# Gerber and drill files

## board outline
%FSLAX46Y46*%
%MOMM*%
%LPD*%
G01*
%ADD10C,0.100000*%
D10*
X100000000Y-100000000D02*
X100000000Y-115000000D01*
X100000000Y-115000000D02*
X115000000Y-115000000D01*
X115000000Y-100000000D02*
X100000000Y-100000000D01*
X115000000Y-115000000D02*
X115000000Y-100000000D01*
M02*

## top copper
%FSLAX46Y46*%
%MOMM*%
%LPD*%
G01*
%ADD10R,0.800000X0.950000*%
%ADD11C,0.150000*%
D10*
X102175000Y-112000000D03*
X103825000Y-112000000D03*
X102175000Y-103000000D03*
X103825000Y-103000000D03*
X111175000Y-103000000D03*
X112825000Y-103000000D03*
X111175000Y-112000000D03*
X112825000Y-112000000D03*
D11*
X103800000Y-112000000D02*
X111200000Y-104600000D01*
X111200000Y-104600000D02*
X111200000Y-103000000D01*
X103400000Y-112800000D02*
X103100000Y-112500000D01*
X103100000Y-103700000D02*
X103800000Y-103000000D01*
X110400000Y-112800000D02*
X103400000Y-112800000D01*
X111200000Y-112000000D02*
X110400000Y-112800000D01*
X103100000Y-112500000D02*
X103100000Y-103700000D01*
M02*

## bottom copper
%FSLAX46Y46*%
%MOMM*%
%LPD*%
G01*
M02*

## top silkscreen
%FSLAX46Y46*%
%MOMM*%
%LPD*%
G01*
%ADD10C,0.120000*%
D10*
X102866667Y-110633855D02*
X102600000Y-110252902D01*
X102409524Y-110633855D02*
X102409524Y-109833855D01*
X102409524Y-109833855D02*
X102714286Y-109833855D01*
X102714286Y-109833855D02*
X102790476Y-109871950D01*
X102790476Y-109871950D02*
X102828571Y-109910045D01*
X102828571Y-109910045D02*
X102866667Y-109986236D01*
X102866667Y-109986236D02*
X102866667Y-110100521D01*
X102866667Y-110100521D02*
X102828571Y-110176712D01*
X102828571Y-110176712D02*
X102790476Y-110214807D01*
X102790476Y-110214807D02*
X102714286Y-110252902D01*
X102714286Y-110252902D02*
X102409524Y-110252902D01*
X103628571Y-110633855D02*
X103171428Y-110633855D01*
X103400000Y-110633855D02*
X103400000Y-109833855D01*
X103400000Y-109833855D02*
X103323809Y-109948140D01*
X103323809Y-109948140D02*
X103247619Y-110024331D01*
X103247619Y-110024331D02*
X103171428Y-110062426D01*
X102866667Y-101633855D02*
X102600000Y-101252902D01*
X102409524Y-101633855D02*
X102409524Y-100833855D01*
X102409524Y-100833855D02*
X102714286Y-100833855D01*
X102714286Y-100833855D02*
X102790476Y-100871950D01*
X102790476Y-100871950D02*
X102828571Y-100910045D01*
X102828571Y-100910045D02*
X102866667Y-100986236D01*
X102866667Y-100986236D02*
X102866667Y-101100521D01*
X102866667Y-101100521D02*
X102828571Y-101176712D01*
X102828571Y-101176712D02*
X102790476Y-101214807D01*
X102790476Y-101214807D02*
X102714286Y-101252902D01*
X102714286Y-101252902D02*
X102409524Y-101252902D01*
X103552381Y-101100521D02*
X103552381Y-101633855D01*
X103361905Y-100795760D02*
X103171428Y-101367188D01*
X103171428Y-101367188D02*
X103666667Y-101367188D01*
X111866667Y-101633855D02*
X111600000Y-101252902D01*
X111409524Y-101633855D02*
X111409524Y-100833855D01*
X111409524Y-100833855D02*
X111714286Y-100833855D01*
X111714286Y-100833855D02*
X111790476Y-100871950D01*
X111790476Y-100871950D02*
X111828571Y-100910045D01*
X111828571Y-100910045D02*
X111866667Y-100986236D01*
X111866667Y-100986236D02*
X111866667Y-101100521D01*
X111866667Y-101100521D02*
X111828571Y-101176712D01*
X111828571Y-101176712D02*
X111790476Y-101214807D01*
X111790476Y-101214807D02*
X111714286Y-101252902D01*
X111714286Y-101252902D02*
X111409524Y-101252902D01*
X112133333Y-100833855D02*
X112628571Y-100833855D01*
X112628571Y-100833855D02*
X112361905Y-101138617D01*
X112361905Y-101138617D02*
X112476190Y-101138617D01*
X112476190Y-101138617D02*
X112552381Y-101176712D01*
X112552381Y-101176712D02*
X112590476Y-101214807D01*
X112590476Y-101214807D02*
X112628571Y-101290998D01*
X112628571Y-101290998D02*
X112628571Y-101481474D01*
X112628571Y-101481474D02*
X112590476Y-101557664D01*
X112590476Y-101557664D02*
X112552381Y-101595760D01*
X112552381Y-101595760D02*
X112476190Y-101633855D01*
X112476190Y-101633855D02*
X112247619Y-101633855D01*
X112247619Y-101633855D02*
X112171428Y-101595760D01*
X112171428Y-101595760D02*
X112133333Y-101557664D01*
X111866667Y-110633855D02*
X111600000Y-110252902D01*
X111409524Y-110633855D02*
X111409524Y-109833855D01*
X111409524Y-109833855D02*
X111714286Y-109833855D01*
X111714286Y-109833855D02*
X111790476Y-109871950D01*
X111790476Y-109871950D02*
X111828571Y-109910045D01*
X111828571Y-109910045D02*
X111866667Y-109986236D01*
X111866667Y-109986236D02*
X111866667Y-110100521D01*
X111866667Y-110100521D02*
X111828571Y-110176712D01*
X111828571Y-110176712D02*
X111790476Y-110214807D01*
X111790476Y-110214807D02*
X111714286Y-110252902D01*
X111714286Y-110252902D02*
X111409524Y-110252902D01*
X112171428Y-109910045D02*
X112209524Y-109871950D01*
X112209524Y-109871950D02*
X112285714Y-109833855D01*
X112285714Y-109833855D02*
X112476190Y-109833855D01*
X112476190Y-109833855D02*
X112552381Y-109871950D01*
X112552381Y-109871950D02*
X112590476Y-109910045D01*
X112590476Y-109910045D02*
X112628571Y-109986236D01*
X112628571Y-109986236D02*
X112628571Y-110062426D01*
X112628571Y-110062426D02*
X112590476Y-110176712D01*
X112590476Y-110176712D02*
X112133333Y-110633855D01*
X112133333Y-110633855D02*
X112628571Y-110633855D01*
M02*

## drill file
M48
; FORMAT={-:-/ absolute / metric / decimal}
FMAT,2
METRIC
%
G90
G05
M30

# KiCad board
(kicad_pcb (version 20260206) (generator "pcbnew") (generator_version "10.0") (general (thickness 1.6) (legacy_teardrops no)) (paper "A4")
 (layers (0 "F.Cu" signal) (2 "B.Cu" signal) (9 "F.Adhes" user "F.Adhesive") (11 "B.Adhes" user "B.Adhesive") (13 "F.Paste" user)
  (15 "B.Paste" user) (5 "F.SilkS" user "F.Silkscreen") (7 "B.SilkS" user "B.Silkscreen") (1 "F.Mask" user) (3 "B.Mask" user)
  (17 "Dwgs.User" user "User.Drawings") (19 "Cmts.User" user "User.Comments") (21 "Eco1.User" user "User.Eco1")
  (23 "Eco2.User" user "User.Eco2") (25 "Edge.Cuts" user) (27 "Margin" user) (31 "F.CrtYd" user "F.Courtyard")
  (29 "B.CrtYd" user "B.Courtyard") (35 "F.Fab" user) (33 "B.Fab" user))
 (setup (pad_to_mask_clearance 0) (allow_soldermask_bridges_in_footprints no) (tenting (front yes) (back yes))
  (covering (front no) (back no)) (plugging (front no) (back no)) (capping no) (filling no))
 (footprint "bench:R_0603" (layer "F.Cu") (at 103 112)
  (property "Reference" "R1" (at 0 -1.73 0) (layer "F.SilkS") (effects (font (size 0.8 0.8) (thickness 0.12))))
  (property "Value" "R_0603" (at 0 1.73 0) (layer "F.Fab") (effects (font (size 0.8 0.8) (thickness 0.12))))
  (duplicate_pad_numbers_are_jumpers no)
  (pad "1" smd rect (at -0.825 0) (size 0.8 0.95) (layers "F.Cu" "F.Mask" "F.Paste"))
  (pad "2" smd rect (at 0.825 0) (size 0.8 0.95) (layers "F.Cu" "F.Mask" "F.Paste") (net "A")))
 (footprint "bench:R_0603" (layer "F.Cu") (at 103 103)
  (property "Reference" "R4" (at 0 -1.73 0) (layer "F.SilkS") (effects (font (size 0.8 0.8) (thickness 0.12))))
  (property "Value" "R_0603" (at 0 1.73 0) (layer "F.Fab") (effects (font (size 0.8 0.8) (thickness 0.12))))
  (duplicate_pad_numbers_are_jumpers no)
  (pad "1" smd rect (at -0.825 0) (size 0.8 0.95) (layers "F.Cu" "F.Mask" "F.Paste"))
  (pad "2" smd rect (at 0.825 0) (size 0.8 0.95) (layers "F.Cu" "F.Mask" "F.Paste") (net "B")))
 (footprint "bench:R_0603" (layer "F.Cu") (at 112 103)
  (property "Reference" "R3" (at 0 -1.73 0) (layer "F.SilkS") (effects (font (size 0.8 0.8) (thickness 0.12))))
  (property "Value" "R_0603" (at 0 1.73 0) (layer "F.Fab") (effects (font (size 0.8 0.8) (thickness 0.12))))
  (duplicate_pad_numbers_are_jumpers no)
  (pad "1" smd rect (at -0.825 0) (size 0.8 0.95) (layers "F.Cu" "F.Mask" "F.Paste") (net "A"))
  (pad "2" smd rect (at 0.825 0) (size 0.8 0.95) (layers "F.Cu" "F.Mask" "F.Paste")))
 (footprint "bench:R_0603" (layer "F.Cu") (at 112 112)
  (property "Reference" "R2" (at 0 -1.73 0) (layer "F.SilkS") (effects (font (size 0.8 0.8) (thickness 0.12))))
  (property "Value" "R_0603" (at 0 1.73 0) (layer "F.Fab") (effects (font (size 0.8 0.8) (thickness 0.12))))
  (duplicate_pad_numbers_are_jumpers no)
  (pad "1" smd rect (at -0.825 0) (size 0.8 0.95) (layers "F.Cu" "F.Mask" "F.Paste") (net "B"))
  (pad "2" smd rect (at 0.825 0) (size 0.8 0.95) (layers "F.Cu" "F.Mask" "F.Paste")))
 (gr_line (start 100 100) (end 100 115) (stroke (width 0.1) (type solid)) (layer "Edge.Cuts"))
 (gr_line (start 100 115) (end 115 115) (stroke (width 0.1) (type solid)) (layer "Edge.Cuts"))
 (gr_line (start 115 100) (end 100 100) (stroke (width 0.1) (type solid)) (layer "Edge.Cuts"))
 (gr_line (start 115 115) (end 115 100) (stroke (width 0.1) (type solid)) (layer "Edge.Cuts"))
 (segment (start 103.8 112) (end 111.2 104.6) (width 0.15) (layer "F.Cu") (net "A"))
 (segment (start 111.2 104.6) (end 111.2 103) (width 0.15) (layer "F.Cu") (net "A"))
 (segment (start 103.4 112.8) (end 103.1 112.5) (width 0.15) (layer "F.Cu") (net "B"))
 (segment (start 103.1 103.7) (end 103.8 103) (width 0.15) (layer "F.Cu") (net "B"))
 (segment (start 110.4 112.8) (end 103.4 112.8) (width 0.15) (layer "F.Cu") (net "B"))
 (segment (start 111.2 112) (end 110.4 112.8) (width 0.15) (layer "F.Cu") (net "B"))
 (segment (start 103.1 112.5) (end 103.1 103.7) (width 0.15) (layer "F.Cu") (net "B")))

